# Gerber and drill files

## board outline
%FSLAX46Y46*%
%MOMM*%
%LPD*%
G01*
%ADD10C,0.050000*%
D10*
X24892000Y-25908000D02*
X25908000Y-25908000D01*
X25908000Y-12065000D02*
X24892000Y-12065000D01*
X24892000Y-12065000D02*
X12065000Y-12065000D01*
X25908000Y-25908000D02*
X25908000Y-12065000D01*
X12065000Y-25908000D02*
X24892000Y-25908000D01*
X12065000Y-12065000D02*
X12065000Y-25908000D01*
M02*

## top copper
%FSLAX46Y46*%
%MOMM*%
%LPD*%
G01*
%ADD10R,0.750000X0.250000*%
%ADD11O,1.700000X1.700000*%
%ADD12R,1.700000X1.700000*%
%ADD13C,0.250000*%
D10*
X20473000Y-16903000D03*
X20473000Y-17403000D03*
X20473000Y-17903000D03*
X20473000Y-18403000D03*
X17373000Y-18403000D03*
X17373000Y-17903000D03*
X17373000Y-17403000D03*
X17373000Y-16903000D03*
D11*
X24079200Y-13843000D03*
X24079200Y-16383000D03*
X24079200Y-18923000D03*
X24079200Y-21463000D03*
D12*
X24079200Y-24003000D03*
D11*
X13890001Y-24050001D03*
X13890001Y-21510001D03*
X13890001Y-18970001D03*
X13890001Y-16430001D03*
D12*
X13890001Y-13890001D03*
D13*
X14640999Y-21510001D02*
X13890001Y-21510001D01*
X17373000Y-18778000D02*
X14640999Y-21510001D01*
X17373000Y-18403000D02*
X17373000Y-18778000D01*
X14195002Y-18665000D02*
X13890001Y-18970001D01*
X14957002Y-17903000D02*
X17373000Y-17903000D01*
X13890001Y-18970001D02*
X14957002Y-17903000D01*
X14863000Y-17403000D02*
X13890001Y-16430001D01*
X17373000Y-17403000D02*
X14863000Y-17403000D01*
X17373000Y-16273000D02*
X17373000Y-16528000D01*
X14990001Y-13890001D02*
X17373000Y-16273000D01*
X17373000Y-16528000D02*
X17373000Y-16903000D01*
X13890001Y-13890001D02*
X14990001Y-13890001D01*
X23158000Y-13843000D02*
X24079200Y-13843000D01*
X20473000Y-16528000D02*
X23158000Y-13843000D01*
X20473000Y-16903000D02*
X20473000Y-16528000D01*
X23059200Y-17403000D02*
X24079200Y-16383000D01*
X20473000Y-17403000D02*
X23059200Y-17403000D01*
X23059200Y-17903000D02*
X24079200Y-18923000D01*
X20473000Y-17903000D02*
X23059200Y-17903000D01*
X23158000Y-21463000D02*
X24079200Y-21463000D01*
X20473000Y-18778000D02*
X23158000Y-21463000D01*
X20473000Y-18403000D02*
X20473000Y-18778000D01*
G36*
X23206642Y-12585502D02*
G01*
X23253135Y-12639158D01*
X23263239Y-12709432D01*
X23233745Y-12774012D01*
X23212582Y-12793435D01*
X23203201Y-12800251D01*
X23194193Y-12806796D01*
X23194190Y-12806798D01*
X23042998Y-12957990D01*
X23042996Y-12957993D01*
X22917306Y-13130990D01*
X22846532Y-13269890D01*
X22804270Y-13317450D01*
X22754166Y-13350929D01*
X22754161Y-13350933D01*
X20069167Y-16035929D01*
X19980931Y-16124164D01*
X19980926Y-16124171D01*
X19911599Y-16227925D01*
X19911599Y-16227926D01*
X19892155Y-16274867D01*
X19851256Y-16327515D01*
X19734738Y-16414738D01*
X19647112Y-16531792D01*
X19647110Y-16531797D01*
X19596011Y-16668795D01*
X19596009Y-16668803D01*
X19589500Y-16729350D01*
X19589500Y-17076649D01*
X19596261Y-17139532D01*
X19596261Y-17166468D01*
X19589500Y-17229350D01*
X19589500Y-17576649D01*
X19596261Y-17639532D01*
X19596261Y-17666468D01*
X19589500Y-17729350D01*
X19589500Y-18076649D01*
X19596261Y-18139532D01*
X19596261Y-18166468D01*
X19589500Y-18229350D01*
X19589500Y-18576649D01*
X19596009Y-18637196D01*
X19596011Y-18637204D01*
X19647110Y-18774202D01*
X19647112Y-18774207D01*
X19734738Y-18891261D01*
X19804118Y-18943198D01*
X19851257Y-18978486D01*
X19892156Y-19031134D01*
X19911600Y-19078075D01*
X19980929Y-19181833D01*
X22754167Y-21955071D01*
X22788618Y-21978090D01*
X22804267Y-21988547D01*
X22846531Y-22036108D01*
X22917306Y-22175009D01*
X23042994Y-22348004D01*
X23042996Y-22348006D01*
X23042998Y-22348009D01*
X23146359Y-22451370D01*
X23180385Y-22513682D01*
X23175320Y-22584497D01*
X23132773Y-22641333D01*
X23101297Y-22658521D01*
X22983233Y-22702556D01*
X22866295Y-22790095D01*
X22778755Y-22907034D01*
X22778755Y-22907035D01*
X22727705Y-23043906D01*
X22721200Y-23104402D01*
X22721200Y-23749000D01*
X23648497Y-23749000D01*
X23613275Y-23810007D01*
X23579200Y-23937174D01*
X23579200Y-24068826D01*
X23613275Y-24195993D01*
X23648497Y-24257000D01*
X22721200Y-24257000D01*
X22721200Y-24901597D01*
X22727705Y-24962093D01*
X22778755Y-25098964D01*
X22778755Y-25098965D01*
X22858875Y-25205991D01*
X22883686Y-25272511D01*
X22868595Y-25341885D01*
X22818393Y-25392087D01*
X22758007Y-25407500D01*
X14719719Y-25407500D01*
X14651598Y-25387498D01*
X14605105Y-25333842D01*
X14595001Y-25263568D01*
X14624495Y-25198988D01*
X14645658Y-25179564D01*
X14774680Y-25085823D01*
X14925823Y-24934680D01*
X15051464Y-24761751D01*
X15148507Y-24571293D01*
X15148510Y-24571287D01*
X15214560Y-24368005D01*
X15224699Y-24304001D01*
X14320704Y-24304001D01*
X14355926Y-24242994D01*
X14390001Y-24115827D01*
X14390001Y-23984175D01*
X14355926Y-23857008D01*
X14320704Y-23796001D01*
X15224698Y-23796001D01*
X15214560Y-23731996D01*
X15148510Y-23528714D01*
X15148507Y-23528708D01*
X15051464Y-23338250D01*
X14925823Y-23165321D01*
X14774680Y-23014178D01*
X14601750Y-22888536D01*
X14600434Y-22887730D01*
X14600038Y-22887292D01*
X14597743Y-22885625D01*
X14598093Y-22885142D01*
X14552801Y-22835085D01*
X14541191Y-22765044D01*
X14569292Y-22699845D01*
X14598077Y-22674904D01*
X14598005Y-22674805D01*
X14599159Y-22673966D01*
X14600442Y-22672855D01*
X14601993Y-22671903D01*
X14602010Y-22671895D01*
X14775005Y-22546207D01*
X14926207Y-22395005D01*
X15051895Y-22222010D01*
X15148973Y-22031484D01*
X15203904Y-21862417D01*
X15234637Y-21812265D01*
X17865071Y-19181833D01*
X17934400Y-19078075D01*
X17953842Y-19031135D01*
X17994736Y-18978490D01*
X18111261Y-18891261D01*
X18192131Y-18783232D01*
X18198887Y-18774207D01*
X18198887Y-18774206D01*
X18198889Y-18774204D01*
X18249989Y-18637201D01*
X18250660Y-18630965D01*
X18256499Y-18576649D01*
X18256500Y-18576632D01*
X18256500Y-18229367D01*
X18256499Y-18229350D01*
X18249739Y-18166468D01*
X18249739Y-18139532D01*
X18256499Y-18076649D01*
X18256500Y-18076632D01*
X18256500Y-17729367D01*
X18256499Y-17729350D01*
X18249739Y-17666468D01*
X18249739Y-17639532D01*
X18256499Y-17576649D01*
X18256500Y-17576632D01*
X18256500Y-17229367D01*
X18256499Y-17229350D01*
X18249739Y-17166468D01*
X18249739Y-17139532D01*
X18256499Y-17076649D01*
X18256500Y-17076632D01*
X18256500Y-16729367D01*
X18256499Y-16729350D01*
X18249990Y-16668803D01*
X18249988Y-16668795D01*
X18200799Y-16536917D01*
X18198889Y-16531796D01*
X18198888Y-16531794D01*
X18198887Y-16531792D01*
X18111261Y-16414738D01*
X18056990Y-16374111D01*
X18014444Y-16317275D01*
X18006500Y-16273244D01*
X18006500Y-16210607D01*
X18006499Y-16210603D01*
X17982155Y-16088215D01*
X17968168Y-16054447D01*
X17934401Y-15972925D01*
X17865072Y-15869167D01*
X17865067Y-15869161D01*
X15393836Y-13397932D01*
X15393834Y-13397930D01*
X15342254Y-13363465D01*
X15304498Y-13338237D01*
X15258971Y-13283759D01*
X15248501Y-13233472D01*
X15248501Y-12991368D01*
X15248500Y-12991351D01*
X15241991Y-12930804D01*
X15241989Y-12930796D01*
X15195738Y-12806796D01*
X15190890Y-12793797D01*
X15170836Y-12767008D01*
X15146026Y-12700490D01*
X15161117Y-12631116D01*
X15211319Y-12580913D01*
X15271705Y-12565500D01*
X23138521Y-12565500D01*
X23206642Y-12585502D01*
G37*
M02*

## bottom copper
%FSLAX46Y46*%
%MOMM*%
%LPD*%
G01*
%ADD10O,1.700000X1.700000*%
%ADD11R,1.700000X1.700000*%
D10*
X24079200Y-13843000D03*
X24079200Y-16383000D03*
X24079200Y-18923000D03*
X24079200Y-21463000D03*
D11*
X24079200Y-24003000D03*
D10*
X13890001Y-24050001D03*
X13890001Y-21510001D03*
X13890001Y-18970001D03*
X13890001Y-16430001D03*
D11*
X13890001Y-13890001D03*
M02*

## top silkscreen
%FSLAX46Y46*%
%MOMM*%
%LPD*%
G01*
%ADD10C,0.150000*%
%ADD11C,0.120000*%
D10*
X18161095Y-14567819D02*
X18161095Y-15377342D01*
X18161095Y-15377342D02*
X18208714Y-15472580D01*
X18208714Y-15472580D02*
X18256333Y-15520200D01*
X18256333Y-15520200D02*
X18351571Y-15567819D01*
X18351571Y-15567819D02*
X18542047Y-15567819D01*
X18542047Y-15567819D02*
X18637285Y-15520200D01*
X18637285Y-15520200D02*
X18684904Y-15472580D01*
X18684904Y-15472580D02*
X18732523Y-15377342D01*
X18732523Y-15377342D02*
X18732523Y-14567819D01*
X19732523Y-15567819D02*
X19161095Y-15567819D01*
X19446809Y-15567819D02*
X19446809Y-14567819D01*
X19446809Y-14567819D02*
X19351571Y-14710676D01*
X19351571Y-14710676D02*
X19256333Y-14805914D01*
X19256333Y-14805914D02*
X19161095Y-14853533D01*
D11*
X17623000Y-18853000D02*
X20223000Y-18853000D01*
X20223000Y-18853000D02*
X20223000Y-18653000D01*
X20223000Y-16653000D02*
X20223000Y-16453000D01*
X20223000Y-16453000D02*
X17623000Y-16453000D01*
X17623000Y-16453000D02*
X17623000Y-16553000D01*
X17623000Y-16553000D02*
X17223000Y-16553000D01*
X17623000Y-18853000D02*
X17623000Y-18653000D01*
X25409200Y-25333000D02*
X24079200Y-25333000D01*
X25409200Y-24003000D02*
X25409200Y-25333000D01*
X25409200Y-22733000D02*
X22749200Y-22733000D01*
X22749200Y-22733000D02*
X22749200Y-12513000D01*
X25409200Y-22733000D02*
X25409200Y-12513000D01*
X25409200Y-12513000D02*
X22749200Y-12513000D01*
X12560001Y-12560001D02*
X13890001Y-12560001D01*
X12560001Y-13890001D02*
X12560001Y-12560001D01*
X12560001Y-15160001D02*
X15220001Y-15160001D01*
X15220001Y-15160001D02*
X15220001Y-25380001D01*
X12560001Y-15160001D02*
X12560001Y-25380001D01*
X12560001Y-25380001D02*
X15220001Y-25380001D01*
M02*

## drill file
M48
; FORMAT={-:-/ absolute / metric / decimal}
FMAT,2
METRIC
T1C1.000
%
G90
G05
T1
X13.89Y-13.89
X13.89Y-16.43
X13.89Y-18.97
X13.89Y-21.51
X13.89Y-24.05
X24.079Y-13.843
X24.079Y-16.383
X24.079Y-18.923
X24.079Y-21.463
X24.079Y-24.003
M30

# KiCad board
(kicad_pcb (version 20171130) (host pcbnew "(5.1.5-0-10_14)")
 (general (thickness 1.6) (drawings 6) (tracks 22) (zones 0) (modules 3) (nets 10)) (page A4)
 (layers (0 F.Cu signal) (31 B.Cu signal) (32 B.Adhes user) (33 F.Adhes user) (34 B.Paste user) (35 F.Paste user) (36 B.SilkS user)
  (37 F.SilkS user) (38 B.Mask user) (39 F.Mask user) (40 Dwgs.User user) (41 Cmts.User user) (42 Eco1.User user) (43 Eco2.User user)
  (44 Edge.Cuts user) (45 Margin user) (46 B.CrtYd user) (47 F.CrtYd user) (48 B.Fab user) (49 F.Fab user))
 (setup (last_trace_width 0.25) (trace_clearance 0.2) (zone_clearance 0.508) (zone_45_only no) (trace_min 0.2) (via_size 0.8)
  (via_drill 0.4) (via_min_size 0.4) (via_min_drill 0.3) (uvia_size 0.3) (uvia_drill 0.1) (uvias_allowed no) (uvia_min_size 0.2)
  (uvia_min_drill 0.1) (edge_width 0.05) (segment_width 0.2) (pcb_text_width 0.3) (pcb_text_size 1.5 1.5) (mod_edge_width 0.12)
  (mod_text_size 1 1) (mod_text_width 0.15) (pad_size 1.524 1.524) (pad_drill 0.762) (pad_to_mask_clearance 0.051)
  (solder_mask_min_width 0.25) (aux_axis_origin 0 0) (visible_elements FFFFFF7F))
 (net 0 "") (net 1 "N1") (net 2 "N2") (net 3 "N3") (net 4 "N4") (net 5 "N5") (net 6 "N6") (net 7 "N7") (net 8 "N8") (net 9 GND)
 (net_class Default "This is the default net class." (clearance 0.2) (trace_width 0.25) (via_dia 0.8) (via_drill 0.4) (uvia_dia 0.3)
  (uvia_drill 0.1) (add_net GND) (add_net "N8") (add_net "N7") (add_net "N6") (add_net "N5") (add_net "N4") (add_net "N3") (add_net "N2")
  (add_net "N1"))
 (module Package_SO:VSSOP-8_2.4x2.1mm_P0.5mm (layer F.Cu) (at 18.923 17.653)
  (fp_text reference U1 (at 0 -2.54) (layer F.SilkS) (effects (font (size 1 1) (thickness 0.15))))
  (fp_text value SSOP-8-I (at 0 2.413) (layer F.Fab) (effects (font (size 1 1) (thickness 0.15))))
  (fp_line (start -1.3 1.2) (end 1.3 1.2) (layer F.SilkS) (width 0.12))
  (fp_line (start 1.3 1.2) (end 1.3 1) (layer F.SilkS) (width 0.12))
  (fp_line (start 1.3 -1) (end 1.3 -1.2) (layer F.SilkS) (width 0.12))
  (fp_line (start 1.3 -1.2) (end -1.3 -1.2) (layer F.SilkS) (width 0.12))
  (fp_line (start -1.3 -1.2) (end -1.3 -1.1) (layer F.SilkS) (width 0.12))
  (fp_line (start -1.3 -1.1) (end -1.7 -1.1) (layer F.SilkS) (width 0.12))
  (fp_line (start -1.3 1.2) (end -1.3 1) (layer F.SilkS) (width 0.12))
  (pad 8 smd rect (at 1.55 -0.75) (size 0.75 0.25) (layers F.Cu F.Paste F.Mask) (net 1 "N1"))
  (pad 7 smd rect (at 1.55 -0.25) (size 0.75 0.25) (layers F.Cu F.Paste F.Mask) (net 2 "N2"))
  (pad 6 smd rect (at 1.55 0.25) (size 0.75 0.25) (layers F.Cu F.Paste F.Mask) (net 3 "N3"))
  (pad 5 smd rect (at 1.55 0.75) (size 0.75 0.25) (layers F.Cu F.Paste F.Mask) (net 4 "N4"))
  (pad 4 smd rect (at -1.55 0.75) (size 0.75 0.25) (layers F.Cu F.Paste F.Mask) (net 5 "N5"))
  (pad 3 smd rect (at -1.55 0.25) (size 0.75 0.25) (layers F.Cu F.Paste F.Mask) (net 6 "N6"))
  (pad 2 smd rect (at -1.55 -0.25) (size 0.75 0.25) (layers F.Cu F.Paste F.Mask) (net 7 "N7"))
  (pad 1 smd rect (at -1.55 -0.75) (size 0.75 0.25) (layers F.Cu F.Paste F.Mask) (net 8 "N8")))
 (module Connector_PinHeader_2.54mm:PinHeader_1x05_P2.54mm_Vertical (layer F.Cu) (at 24.0792 24.003 180)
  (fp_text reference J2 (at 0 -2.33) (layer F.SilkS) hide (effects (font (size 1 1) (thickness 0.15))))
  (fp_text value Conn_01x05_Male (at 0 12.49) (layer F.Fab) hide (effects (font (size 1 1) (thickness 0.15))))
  (fp_line (start -1.33 -1.33) (end 0 -1.33) (layer F.SilkS) (width 0.12))
  (fp_line (start -1.33 0) (end -1.33 -1.33) (layer F.SilkS) (width 0.12))
  (fp_line (start -1.33 1.27) (end 1.33 1.27) (layer F.SilkS) (width 0.12))
  (fp_line (start 1.33 1.27) (end 1.33 11.49) (layer F.SilkS) (width 0.12))
  (fp_line (start -1.33 1.27) (end -1.33 11.49) (layer F.SilkS) (width 0.12))
  (fp_line (start -1.33 11.49) (end 1.33 11.49) (layer F.SilkS) (width 0.12))
  (pad 5 thru_hole oval (at 0 10.16 180) (size 1.7 1.7) (drill 1) (layers *.Cu *.Mask) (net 1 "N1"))
  (pad 4 thru_hole oval (at 0 7.62 180) (size 1.7 1.7) (drill 1) (layers *.Cu *.Mask) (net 2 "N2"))
  (pad 3 thru_hole oval (at 0 5.08 180) (size 1.7 1.7) (drill 1) (layers *.Cu *.Mask) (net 3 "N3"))
  (pad 2 thru_hole oval (at 0 2.54 180) (size 1.7 1.7) (drill 1) (layers *.Cu *.Mask) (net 4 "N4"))
  (pad 1 thru_hole rect (at 0 0 180) (size 1.7 1.7) (drill 1) (layers *.Cu *.Mask) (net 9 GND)))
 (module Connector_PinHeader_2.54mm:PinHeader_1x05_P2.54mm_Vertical (layer F.Cu) (at 13.890001 13.890001)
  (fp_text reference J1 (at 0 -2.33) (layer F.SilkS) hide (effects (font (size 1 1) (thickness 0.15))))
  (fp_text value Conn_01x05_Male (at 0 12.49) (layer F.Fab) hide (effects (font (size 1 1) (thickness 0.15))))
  (fp_line (start -1.33 -1.33) (end 0 -1.33) (layer F.SilkS) (width 0.12))
  (fp_line (start -1.33 0) (end -1.33 -1.33) (layer F.SilkS) (width 0.12))
  (fp_line (start -1.33 1.27) (end 1.33 1.27) (layer F.SilkS) (width 0.12))
  (fp_line (start 1.33 1.27) (end 1.33 11.49) (layer F.SilkS) (width 0.12))
  (fp_line (start -1.33 1.27) (end -1.33 11.49) (layer F.SilkS) (width 0.12))
  (fp_line (start -1.33 11.49) (end 1.33 11.49) (layer F.SilkS) (width 0.12))
  (pad 5 thru_hole oval (at 0 10.16) (size 1.7 1.7) (drill 1) (layers *.Cu *.Mask) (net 9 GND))
  (pad 4 thru_hole oval (at 0 7.62) (size 1.7 1.7) (drill 1) (layers *.Cu *.Mask) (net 5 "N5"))
  (pad 3 thru_hole oval (at 0 5.08) (size 1.7 1.7) (drill 1) (layers *.Cu *.Mask) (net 6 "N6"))
  (pad 2 thru_hole oval (at 0 2.54) (size 1.7 1.7) (drill 1) (layers *.Cu *.Mask) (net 7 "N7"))
  (pad 1 thru_hole rect (at 0 0) (size 1.7 1.7) (drill 1) (layers *.Cu *.Mask) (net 8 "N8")))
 (gr_line (start 24.892 25.908) (end 25.908 25.908) (layer Edge.Cuts) (width 0.05))
 (gr_line (start 25.908 12.065) (end 24.892 12.065) (layer Edge.Cuts) (width 0.05))
 (gr_line (start 24.892 12.065) (end 12.065 12.065) (layer Edge.Cuts) (width 0.05))
 (gr_line (start 25.908 25.908) (end 25.908 12.065) (layer Edge.Cuts) (width 0.05))
 (gr_line (start 12.065 25.908) (end 24.892 25.908) (layer Edge.Cuts) (width 0.05))
 (gr_line (start 12.065 12.065) (end 12.065 25.908) (layer Edge.Cuts) (width 0.05))
 (segment (start 14.640999 21.510001) (end 13.890001 21.510001) (width 0.25) (layer F.Cu) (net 5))
 (segment (start 17.373 18.778) (end 14.640999 21.510001) (width 0.25) (layer F.Cu) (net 5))
 (segment (start 17.373 18.403) (end 17.373 18.778) (width 0.25) (layer F.Cu) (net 5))
 (segment (start 14.195002 18.665) (end 13.890001 18.970001) (width 0.25) (layer F.Cu) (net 6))
 (segment (start 14.957002 17.903) (end 17.373 17.903) (width 0.25) (layer F.Cu) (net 6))
 (segment (start 13.890001 18.970001) (end 14.957002 17.903) (width 0.25) (layer F.Cu) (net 6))
 (segment (start 14.863 17.403) (end 13.890001 16.430001) (width 0.25) (layer F.Cu) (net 7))
 (segment (start 17.373 17.403) (end 14.863 17.403) (width 0.25) (layer F.Cu) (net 7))
 (segment (start 17.373 16.273) (end 17.373 16.528) (width 0.25) (layer F.Cu) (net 8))
 (segment (start 14.990001 13.890001) (end 17.373 16.273) (width 0.25) (layer F.Cu) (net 8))
 (segment (start 17.373 16.528) (end 17.373 16.903) (width 0.25) (layer F.Cu) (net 8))
 (segment (start 13.890001 13.890001) (end 14.990001 13.890001) (width 0.25) (layer F.Cu) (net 8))
 (segment (start 23.158 13.843) (end 24.0792 13.843) (width 0.25) (layer F.Cu) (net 1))
 (segment (start 20.473 16.528) (end 23.158 13.843) (width 0.25) (layer F.Cu) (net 1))
 (segment (start 20.473 16.903) (end 20.473 16.528) (width 0.25) (layer F.Cu) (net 1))
 (segment (start 23.0592 17.403) (end 24.0792 16.383) (width 0.25) (layer F.Cu) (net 2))
 (segment (start 20.473 17.403) (end 23.0592 17.403) (width 0.25) (layer F.Cu) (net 2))
 (segment (start 23.0592 17.903) (end 24.0792 18.923) (width 0.25) (layer F.Cu) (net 3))
 (segment (start 20.473 17.903) (end 23.0592 17.903) (width 0.25) (layer F.Cu) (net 3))
 (segment (start 23.158 21.463) (end 24.0792 21.463) (width 0.25) (layer F.Cu) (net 4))
 (segment (start 20.473 18.778) (end 23.158 21.463) (width 0.25) (layer F.Cu) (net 4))
 (segment (start 20.473 18.403) (end 20.473 18.778) (width 0.25) (layer F.Cu) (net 4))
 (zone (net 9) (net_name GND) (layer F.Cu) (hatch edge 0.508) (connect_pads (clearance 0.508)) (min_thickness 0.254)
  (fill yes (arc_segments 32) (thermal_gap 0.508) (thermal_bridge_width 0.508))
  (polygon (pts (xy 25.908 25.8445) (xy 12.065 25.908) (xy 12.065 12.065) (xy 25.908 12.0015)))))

